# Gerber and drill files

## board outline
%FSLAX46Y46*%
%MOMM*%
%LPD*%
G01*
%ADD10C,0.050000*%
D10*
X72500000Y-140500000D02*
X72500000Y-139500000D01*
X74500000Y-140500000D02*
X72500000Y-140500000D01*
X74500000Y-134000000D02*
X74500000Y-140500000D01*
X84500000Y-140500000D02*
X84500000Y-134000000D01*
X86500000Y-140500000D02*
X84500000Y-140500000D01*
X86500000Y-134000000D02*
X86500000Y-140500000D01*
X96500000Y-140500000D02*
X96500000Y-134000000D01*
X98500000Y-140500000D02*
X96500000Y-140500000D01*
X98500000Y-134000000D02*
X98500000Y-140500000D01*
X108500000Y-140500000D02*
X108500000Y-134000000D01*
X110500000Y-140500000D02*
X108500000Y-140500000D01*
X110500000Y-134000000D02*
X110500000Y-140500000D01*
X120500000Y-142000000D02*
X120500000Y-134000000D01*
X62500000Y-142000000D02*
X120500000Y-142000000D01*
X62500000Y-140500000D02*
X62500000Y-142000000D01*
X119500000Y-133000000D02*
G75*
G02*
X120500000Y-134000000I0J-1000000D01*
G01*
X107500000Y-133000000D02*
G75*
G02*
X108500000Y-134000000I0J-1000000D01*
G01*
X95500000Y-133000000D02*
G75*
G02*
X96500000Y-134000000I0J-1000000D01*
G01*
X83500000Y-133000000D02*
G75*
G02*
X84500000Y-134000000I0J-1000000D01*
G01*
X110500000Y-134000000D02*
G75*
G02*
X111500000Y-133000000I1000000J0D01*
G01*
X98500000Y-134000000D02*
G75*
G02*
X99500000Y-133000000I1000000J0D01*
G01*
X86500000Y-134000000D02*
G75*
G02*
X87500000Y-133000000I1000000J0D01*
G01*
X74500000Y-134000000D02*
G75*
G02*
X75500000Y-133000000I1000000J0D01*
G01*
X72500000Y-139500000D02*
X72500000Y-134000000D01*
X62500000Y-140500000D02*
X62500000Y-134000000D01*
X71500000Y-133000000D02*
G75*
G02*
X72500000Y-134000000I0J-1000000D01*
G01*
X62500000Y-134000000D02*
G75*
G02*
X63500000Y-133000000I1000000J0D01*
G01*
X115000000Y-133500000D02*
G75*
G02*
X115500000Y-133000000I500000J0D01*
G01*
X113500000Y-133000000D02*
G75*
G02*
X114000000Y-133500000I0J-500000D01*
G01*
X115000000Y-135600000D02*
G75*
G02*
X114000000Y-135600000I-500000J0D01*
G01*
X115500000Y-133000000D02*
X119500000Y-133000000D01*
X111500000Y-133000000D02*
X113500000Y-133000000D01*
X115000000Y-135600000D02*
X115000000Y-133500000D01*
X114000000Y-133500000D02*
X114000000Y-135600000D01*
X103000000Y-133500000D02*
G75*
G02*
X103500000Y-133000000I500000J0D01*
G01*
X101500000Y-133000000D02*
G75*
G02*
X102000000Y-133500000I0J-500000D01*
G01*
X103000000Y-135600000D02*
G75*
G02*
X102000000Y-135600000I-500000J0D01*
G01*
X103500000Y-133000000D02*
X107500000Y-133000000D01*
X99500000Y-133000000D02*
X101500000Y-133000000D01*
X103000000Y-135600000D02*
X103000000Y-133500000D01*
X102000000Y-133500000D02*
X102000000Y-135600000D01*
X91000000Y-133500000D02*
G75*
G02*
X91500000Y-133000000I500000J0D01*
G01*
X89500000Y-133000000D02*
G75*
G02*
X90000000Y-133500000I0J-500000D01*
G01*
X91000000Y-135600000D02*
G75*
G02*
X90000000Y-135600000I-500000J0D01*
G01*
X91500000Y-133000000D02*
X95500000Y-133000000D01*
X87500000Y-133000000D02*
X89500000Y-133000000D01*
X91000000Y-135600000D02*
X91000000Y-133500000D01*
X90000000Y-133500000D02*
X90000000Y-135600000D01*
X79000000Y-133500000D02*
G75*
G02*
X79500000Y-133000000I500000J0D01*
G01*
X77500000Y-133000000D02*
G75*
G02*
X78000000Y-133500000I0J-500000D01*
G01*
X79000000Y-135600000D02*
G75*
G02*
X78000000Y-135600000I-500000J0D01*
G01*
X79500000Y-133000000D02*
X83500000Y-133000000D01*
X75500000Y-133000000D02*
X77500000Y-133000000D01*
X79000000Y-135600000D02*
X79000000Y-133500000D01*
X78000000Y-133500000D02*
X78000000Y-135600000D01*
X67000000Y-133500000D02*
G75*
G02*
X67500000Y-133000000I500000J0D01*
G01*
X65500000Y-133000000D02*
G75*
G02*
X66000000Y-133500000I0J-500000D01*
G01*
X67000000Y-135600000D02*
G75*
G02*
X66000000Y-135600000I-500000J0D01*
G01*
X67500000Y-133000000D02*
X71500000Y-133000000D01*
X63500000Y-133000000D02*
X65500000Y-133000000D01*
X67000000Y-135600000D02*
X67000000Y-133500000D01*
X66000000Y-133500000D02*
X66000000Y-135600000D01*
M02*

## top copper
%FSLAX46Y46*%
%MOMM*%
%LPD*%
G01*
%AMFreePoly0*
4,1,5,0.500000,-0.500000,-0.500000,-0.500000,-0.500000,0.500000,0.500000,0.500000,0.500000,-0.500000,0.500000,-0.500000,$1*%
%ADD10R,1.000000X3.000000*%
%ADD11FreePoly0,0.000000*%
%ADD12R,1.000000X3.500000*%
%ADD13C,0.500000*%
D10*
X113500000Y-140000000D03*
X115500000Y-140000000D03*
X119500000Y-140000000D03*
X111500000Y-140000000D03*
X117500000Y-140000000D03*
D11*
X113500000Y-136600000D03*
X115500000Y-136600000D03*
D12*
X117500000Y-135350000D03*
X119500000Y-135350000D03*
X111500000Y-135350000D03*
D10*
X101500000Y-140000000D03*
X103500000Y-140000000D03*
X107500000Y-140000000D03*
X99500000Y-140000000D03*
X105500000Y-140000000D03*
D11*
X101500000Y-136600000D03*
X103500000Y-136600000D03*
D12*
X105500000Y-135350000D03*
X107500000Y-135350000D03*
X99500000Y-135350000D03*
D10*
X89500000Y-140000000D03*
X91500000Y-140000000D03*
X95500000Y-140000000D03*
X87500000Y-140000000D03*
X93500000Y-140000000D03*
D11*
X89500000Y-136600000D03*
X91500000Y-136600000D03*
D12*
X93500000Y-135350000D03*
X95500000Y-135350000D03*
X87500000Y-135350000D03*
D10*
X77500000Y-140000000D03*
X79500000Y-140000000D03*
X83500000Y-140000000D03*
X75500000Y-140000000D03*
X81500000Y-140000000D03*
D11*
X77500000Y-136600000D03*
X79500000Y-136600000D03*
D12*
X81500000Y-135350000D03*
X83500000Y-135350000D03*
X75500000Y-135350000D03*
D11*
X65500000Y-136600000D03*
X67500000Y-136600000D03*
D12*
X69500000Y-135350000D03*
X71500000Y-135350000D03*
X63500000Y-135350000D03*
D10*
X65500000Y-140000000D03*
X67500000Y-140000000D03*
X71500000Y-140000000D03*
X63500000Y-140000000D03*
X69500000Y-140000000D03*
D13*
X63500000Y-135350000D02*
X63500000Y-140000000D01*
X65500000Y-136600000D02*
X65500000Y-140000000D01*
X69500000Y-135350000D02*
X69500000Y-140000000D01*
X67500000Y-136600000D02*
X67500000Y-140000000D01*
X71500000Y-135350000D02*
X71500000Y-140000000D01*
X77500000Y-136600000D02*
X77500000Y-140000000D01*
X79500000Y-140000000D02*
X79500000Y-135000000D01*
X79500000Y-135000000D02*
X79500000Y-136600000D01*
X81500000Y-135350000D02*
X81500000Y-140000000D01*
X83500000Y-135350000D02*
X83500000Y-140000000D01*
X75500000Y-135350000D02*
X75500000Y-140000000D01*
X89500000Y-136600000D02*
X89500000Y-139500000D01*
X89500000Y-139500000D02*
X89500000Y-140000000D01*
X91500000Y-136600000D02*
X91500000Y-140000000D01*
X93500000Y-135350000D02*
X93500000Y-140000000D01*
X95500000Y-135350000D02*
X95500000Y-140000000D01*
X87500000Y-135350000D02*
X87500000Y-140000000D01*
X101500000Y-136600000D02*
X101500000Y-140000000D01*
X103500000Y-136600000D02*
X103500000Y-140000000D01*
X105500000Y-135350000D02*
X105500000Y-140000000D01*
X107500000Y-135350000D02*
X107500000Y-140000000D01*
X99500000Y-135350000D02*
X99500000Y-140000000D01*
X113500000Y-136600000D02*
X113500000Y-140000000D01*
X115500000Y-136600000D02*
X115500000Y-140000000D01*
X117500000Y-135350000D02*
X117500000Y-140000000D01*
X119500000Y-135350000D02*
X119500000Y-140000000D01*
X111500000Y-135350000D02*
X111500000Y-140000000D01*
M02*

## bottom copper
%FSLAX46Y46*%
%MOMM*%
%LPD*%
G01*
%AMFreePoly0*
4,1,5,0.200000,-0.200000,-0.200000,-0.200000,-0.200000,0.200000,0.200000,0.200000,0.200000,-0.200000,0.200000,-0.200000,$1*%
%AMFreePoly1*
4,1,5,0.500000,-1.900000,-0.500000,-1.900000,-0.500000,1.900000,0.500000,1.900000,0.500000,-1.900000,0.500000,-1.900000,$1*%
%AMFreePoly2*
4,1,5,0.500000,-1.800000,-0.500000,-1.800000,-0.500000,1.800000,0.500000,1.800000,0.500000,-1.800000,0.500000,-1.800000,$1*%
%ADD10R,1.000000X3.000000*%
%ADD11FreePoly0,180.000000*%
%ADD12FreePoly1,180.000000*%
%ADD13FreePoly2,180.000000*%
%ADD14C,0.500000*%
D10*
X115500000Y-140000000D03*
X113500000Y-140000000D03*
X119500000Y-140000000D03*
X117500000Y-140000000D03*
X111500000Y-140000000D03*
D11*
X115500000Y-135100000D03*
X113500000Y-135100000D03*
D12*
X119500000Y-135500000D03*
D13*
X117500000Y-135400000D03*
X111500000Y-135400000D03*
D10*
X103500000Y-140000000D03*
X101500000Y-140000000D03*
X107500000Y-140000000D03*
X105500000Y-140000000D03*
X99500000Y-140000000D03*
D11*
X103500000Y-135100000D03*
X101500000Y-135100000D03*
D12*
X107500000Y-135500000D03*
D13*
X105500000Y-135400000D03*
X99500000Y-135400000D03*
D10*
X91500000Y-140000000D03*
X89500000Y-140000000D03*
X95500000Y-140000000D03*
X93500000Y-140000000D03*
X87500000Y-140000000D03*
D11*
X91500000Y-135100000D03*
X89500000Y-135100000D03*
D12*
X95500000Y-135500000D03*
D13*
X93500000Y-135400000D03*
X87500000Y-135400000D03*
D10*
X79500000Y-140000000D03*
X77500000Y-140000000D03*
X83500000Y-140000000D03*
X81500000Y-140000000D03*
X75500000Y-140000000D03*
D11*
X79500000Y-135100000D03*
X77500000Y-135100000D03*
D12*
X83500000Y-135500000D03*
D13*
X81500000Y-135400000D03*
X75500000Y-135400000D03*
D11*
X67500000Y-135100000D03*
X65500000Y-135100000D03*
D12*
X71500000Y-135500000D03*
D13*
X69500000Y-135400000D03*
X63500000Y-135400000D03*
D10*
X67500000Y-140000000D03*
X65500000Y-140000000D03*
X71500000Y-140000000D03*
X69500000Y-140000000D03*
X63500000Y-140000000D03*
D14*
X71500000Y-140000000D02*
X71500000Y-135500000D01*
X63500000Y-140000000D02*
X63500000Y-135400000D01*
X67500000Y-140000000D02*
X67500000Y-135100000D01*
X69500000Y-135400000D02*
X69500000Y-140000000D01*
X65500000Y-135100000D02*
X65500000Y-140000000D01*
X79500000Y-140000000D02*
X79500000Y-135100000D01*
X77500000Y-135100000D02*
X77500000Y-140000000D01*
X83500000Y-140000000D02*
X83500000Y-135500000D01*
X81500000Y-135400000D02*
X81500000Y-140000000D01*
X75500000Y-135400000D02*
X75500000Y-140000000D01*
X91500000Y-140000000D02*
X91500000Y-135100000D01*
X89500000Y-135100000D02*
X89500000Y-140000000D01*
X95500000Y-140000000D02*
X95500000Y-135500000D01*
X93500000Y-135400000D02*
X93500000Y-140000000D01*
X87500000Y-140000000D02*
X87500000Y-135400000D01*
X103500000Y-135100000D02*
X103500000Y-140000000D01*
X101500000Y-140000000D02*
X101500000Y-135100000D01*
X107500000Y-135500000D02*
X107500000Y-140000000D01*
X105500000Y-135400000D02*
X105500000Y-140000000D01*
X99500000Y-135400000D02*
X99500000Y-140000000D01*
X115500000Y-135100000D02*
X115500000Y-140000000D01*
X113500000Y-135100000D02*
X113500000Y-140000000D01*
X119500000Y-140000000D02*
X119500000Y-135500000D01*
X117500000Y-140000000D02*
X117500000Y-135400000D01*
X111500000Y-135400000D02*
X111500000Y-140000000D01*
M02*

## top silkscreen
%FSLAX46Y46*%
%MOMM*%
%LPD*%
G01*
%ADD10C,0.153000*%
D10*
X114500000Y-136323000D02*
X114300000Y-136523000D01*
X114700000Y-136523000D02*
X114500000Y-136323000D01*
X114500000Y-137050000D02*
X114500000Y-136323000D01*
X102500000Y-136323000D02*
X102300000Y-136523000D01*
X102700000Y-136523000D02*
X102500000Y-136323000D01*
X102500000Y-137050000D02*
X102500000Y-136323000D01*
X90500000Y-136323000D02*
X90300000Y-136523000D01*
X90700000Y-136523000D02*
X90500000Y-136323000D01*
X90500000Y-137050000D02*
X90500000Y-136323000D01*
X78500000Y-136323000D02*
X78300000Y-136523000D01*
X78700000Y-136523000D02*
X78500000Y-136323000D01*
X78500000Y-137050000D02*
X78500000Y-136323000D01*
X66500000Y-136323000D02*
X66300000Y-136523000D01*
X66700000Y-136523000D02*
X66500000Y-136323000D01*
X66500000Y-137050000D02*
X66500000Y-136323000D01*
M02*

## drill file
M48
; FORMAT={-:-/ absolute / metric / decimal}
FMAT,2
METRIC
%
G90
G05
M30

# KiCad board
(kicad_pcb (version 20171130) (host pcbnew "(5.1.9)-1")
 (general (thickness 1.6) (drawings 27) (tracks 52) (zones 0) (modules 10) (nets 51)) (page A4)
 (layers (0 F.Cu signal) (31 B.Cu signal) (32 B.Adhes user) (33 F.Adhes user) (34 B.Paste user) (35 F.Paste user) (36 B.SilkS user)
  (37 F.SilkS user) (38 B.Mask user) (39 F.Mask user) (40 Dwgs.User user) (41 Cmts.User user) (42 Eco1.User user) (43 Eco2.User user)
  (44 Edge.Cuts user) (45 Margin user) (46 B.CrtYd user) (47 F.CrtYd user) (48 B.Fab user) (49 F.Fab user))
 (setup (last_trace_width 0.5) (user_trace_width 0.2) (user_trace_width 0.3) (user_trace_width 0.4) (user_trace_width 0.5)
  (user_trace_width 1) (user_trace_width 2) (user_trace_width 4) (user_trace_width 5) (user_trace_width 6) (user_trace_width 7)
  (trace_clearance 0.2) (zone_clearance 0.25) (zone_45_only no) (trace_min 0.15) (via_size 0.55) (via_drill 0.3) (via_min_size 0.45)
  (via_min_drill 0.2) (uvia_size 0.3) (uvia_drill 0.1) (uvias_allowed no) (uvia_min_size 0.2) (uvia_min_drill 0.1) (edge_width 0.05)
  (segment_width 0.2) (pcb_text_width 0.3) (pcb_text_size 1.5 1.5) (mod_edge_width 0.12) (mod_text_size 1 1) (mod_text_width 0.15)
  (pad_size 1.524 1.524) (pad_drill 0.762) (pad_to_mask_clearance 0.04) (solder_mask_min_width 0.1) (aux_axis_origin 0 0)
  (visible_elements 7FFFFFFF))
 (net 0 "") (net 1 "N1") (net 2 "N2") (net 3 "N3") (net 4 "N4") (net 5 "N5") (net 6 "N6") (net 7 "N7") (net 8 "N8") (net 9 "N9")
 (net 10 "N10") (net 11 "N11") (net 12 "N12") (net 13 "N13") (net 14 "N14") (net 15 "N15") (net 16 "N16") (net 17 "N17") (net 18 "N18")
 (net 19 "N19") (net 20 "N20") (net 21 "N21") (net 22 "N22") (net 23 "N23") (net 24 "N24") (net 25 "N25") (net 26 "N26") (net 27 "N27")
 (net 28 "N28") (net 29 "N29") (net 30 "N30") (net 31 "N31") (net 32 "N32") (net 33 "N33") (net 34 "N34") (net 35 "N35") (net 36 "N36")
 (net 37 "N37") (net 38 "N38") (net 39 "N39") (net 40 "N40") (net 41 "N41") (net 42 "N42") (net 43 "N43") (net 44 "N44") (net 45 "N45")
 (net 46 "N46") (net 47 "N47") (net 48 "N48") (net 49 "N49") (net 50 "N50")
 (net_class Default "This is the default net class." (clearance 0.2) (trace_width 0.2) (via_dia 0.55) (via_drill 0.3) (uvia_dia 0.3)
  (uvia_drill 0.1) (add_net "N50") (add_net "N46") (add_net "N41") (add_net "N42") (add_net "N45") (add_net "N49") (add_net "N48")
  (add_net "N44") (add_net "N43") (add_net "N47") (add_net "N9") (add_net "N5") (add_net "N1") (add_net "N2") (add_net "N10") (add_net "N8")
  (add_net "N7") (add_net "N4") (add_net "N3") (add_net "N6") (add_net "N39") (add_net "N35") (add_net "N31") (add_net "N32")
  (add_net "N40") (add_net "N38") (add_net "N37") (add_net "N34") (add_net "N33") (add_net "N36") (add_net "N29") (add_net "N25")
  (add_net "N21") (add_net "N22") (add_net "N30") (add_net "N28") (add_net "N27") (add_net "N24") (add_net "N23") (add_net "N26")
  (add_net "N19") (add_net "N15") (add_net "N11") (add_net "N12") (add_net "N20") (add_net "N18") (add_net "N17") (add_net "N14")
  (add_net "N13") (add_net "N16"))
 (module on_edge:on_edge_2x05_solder (layer F.Cu) (at 115.5 140)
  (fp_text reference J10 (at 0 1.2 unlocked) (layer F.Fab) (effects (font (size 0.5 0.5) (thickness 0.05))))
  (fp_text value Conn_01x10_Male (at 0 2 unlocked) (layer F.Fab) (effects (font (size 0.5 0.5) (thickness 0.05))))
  (pad 2 smd rect (at -2 0) (size 1 3) (layers F.Cu F.Mask) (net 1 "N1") (zone_connect 0))
  (pad 3 smd rect (at 0 0) (size 1 3) (layers F.Cu F.Mask) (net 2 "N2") (zone_connect 0))
  (pad 8 smd rect (at 0 0) (size 1 3) (layers B.Cu B.Mask) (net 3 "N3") (zone_connect 0))
  (pad 7 smd rect (at -2 0) (size 1 3) (layers B.Cu B.Mask) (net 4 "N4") (zone_connect 0))
  (pad 10 smd rect (at 4 0) (size 1 3) (layers B.Cu B.Mask) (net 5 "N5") (zone_connect 0))
  (pad 9 smd rect (at 2 0) (size 1 3) (layers B.Cu B.Mask) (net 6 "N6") (zone_connect 0))
  (pad 6 smd rect (at -4 0) (size 1 3) (layers B.Cu B.Mask) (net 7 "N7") (zone_connect 0))
  (pad 5 smd rect (at 4 0 180) (size 1 3) (layers F.Cu F.Mask) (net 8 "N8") (zone_connect 0))
  (pad 1 smd rect (at -4 0 180) (size 1 3) (layers F.Cu F.Mask) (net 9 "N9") (zone_connect 0))
  (pad 4 smd rect (at 2 0 180) (size 1 3) (layers F.Cu F.Mask) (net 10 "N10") (zone_connect 0)))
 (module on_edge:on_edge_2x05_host (layer F.Cu) (at 115.5 133)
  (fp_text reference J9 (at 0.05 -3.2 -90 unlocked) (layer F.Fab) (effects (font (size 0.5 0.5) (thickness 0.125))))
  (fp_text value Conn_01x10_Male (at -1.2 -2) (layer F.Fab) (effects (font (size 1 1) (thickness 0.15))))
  (fp_arc (start 0 0.5) (end 0 0) (angle -90) (layer Edge.Cuts) (width 0.05))
  (fp_arc (start -2 0.5) (end -1.5 0.5) (angle -90) (layer Edge.Cuts) (width 0.05))
  (fp_arc (start -1 2.6) (end -1.5 2.6) (angle -180) (layer Edge.Cuts) (width 0.05))
  (fp_line (start 0 0) (end 4 0) (layer Edge.Cuts) (width 0.05))
  (fp_line (start -4 0) (end -2 0) (layer Edge.Cuts) (width 0.05))
  (fp_line (start -0.5 2.6) (end -0.5 0.5) (layer Edge.Cuts) (width 0.05))
  (fp_line (start -1.5 0.5) (end -1.5 2.6) (layer Edge.Cuts) (width 0.05))
  (fp_line (start -1 3.323) (end -1.2 3.523) (layer F.SilkS) (width 0.153))
  (fp_line (start -0.8 3.523) (end -1 3.323) (layer F.SilkS) (width 0.153))
  (fp_line (start -1 4.05) (end -1 3.323) (layer F.SilkS) (width 0.153))
  (pad 2 smd custom (at -2 3.6) (size 1 1) (layers F.Cu F.Mask) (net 1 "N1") (zone_connect 0) (options (clearance outline) (anchor rect))
   (primitives))
  (pad 3 smd custom (at 0 3.6) (size 1 1) (layers F.Cu F.Mask) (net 2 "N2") (zone_connect 0) (options (clearance outline) (anchor rect))
   (primitives))
  (pad 8 smd custom (at 0 2.1 180) (size 0.4 0.4) (layers B.Cu B.Mask) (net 3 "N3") (zone_connect 0)
   (options (clearance outline) (anchor rect)) (primitives))
  (pad 7 smd custom (at -2 2.1 180) (size 0.4 0.4) (layers B.Cu B.Mask) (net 4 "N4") (zone_connect 0)
   (options (clearance outline) (anchor rect)) (primitives))
  (pad 4 smd rect (at 2 2.35) (size 1 3.5) (layers F.Cu F.Mask) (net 10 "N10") (zone_connect 0))
  (pad 10 smd custom (at 4 2.5 180) (size 1 3.8) (layers B.Cu B.Mask) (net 5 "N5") (zone_connect 0)
   (options (clearance outline) (anchor rect)) (primitives))
  (pad 9 smd custom (at 2 2.4 180) (size 1 3.6) (layers B.Cu B.Mask) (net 6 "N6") (zone_connect 0)
   (options (clearance outline) (anchor rect)) (primitives))
  (pad 6 smd custom (at -4 2.4 180) (size 1 3.6) (layers B.Cu B.Mask) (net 7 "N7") (zone_connect 0)
   (options (clearance outline) (anchor rect)) (primitives))
  (pad 5 smd rect (at 4 2.35) (size 1 3.5) (layers F.Cu F.Mask) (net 8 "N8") (zone_connect 0))
  (pad 1 smd rect (at -4 2.35) (size 1 3.5) (layers F.Cu F.Mask) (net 9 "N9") (zone_connect 0)))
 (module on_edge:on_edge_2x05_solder (layer F.Cu) (at 103.5 140)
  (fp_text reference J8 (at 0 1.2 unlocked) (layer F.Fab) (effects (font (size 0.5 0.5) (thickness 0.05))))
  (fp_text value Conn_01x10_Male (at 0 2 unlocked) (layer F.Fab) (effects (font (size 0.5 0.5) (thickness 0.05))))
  (pad 2 smd rect (at -2 0) (size 1 3) (layers F.Cu F.Mask) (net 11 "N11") (zone_connect 0))
  (pad 3 smd rect (at 0 0) (size 1 3) (layers F.Cu F.Mask) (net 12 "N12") (zone_connect 0))
  (pad 8 smd rect (at 0 0) (size 1 3) (layers B.Cu B.Mask) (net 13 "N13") (zone_connect 0))
  (pad 7 smd rect (at -2 0) (size 1 3) (layers B.Cu B.Mask) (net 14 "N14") (zone_connect 0))
  (pad 10 smd rect (at 4 0) (size 1 3) (layers B.Cu B.Mask) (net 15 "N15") (zone_connect 0))
  (pad 9 smd rect (at 2 0) (size 1 3) (layers B.Cu B.Mask) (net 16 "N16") (zone_connect 0))
  (pad 6 smd rect (at -4 0) (size 1 3) (layers B.Cu B.Mask) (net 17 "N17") (zone_connect 0))
  (pad 5 smd rect (at 4 0 180) (size 1 3) (layers F.Cu F.Mask) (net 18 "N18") (zone_connect 0))
  (pad 1 smd rect (at -4 0 180) (size 1 3) (layers F.Cu F.Mask) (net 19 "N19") (zone_connect 0))
  (pad 4 smd rect (at 2 0 180) (size 1 3) (layers F.Cu F.Mask) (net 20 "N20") (zone_connect 0)))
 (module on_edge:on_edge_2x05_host (layer F.Cu) (at 103.5 133)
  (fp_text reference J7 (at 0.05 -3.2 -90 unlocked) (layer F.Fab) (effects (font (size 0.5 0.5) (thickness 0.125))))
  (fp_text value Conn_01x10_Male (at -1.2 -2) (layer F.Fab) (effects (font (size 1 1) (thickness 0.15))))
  (fp_arc (start 0 0.5) (end 0 0) (angle -90) (layer Edge.Cuts) (width 0.05))
  (fp_arc (start -2 0.5) (end -1.5 0.5) (angle -90) (layer Edge.Cuts) (width 0.05))
  (fp_arc (start -1 2.6) (end -1.5 2.6) (angle -180) (layer Edge.Cuts) (width 0.05))
  (fp_line (start 0 0) (end 4 0) (layer Edge.Cuts) (width 0.05))
  (fp_line (start -4 0) (end -2 0) (layer Edge.Cuts) (width 0.05))
  (fp_line (start -0.5 2.6) (end -0.5 0.5) (layer Edge.Cuts) (width 0.05))
  (fp_line (start -1.5 0.5) (end -1.5 2.6) (layer Edge.Cuts) (width 0.05))
  (fp_line (start -1 3.323) (end -1.2 3.523) (layer F.SilkS) (width 0.153))
  (fp_line (start -0.8 3.523) (end -1 3.323) (layer F.SilkS) (width 0.153))
  (fp_line (start -1 4.05) (end -1 3.323) (layer F.SilkS) (width 0.153))
  (pad 2 smd custom (at -2 3.6) (size 1 1) (layers F.Cu F.Mask) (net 11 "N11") (zone_connect 0) (options (clearance outline) (anchor rect))
   (primitives))
  (pad 3 smd custom (at 0 3.6) (size 1 1) (layers F.Cu F.Mask) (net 12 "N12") (zone_connect 0) (options (clearance outline) (anchor rect))
   (primitives))
  (pad 8 smd custom (at 0 2.1 180) (size 0.4 0.4) (layers B.Cu B.Mask) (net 13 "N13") (zone_connect 0)
   (options (clearance outline) (anchor rect)) (primitives))
  (pad 7 smd custom (at -2 2.1 180) (size 0.4 0.4) (layers B.Cu B.Mask) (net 14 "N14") (zone_connect 0)
   (options (clearance outline) (anchor rect)) (primitives))
  (pad 4 smd rect (at 2 2.35) (size 1 3.5) (layers F.Cu F.Mask) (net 20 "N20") (zone_connect 0))
  (pad 10 smd custom (at 4 2.5 180) (size 1 3.8) (layers B.Cu B.Mask) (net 15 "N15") (zone_connect 0)
   (options (clearance outline) (anchor rect)) (primitives))
  (pad 9 smd custom (at 2 2.4 180) (size 1 3.6) (layers B.Cu B.Mask) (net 16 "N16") (zone_connect 0)
   (options (clearance outline) (anchor rect)) (primitives))
  (pad 6 smd custom (at -4 2.4 180) (size 1 3.6) (layers B.Cu B.Mask) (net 17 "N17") (zone_connect 0)
   (options (clearance outline) (anchor rect)) (primitives))
  (pad 5 smd rect (at 4 2.35) (size 1 3.5) (layers F.Cu F.Mask) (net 18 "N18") (zone_connect 0))
  (pad 1 smd rect (at -4 2.35) (size 1 3.5) (layers F.Cu F.Mask) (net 19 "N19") (zone_connect 0)))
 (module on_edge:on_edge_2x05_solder (layer F.Cu) (at 91.5 140)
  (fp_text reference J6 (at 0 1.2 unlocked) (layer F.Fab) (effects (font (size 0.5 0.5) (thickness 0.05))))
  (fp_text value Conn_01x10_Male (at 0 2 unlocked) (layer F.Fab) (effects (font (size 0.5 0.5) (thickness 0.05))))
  (pad 2 smd rect (at -2 0) (size 1 3) (layers F.Cu F.Mask) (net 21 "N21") (zone_connect 0))
  (pad 3 smd rect (at 0 0) (size 1 3) (layers F.Cu F.Mask) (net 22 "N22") (zone_connect 0))
  (pad 8 smd rect (at 0 0) (size 1 3) (layers B.Cu B.Mask) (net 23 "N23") (zone_connect 0))
  (pad 7 smd rect (at -2 0) (size 1 3) (layers B.Cu B.Mask) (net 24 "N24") (zone_connect 0))
  (pad 10 smd rect (at 4 0) (size 1 3) (layers B.Cu B.Mask) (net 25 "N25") (zone_connect 0))
  (pad 9 smd rect (at 2 0) (size 1 3) (layers B.Cu B.Mask) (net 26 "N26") (zone_connect 0))
  (pad 6 smd rect (at -4 0) (size 1 3) (layers B.Cu B.Mask) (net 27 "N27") (zone_connect 0))
  (pad 5 smd rect (at 4 0 180) (size 1 3) (layers F.Cu F.Mask) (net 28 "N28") (zone_connect 0))
  (pad 1 smd rect (at -4 0 180) (size 1 3) (layers F.Cu F.Mask) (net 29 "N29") (zone_connect 0))
  (pad 4 smd rect (at 2 0 180) (size 1 3) (layers F.Cu F.Mask) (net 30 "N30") (zone_connect 0)))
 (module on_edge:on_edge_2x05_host (layer F.Cu) (at 91.5 133)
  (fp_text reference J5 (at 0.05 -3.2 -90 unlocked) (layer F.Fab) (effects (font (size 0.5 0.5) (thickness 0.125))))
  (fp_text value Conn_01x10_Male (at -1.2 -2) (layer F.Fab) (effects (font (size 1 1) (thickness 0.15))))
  (fp_arc (start 0 0.5) (end 0 0) (angle -90) (layer Edge.Cuts) (width 0.05))
  (fp_arc (start -2 0.5) (end -1.5 0.5) (angle -90) (layer Edge.Cuts) (width 0.05))
  (fp_arc (start -1 2.6) (end -1.5 2.6) (angle -180) (layer Edge.Cuts) (width 0.05))
  (fp_line (start 0 0) (end 4 0) (layer Edge.Cuts) (width 0.05))
  (fp_line (start -4 0) (end -2 0) (layer Edge.Cuts) (width 0.05))
  (fp_line (start -0.5 2.6) (end -0.5 0.5) (layer Edge.Cuts) (width 0.05))
  (fp_line (start -1.5 0.5) (end -1.5 2.6) (layer Edge.Cuts) (width 0.05))
  (fp_line (start -1 3.323) (end -1.2 3.523) (layer F.SilkS) (width 0.153))
  (fp_line (start -0.8 3.523) (end -1 3.323) (layer F.SilkS) (width 0.153))
  (fp_line (start -1 4.05) (end -1 3.323) (layer F.SilkS) (width 0.153))
  (pad 2 smd custom (at -2 3.6) (size 1 1) (layers F.Cu F.Mask) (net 21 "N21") (zone_connect 0) (options (clearance outline) (anchor rect))
   (primitives))
  (pad 3 smd custom (at 0 3.6) (size 1 1) (layers F.Cu F.Mask) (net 22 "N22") (zone_connect 0) (options (clearance outline) (anchor rect))
   (primitives))
  (pad 8 smd custom (at 0 2.1 180) (size 0.4 0.4) (layers B.Cu B.Mask) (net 23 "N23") (zone_connect 0)
   (options (clearance outline) (anchor rect)) (primitives))
  (pad 7 smd custom (at -2 2.1 180) (size 0.4 0.4) (layers B.Cu B.Mask) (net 24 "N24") (zone_connect 0)
   (options (clearance outline) (anchor rect)) (primitives))
  (pad 4 smd rect (at 2 2.35) (size 1 3.5) (layers F.Cu F.Mask) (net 30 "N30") (zone_connect 0))
  (pad 10 smd custom (at 4 2.5 180) (size 1 3.8) (layers B.Cu B.Mask) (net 25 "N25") (zone_connect 0)
   (options (clearance outline) (anchor rect)) (primitives))
  (pad 9 smd custom (at 2 2.4 180) (size 1 3.6) (layers B.Cu B.Mask) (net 26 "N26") (zone_connect 0)
   (options (clearance outline) (anchor rect)) (primitives))
  (pad 6 smd custom (at -4 2.4 180) (size 1 3.6) (layers B.Cu B.Mask) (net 27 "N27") (zone_connect 0)
   (options (clearance outline) (anchor rect)) (primitives))
  (pad 5 smd rect (at 4 2.35) (size 1 3.5) (layers F.Cu F.Mask) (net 28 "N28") (zone_connect 0))
  (pad 1 smd rect (at -4 2.35) (size 1 3.5) (layers F.Cu F.Mask) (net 29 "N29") (zone_connect 0)))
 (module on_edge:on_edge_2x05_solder (layer F.Cu) (at 79.5 140)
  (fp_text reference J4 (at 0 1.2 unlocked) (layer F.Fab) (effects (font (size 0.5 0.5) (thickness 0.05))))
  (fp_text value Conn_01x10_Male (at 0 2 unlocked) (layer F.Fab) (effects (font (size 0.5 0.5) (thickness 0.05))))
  (pad 2 smd rect (at -2 0) (size 1 3) (layers F.Cu F.Mask) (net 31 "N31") (zone_connect 0))
  (pad 3 smd rect (at 0 0) (size 1 3) (layers F.Cu F.Mask) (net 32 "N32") (zone_connect 0))
  (pad 8 smd rect (at 0 0) (size 1 3) (layers B.Cu B.Mask) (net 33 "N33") (zone_connect 0))
  (pad 7 smd rect (at -2 0) (size 1 3) (layers B.Cu B.Mask) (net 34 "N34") (zone_connect 0))
  (pad 10 smd rect (at 4 0) (size 1 3) (layers B.Cu B.Mask) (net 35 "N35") (zone_connect 0))
  (pad 9 smd rect (at 2 0) (size 1 3) (layers B.Cu B.Mask) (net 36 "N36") (zone_connect 0))
  (pad 6 smd rect (at -4 0) (size 1 3) (layers B.Cu B.Mask) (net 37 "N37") (zone_connect 0))
  (pad 5 smd rect (at 4 0 180) (size 1 3) (layers F.Cu F.Mask) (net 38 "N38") (zone_connect 0))
  (pad 1 smd rect (at -4 0 180) (size 1 3) (layers F.Cu F.Mask) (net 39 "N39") (zone_connect 0))
  (pad 4 smd rect (at 2 0 180) (size 1 3) (layers F.Cu F.Mask) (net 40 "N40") (zone_connect 0)))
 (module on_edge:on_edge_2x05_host (layer F.Cu) (at 79.5 133)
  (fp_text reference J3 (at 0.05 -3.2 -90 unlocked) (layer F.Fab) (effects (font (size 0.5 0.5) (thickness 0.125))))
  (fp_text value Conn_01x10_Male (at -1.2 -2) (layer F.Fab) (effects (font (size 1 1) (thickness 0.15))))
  (fp_arc (start 0 0.5) (end 0 0) (angle -90) (layer Edge.Cuts) (width 0.05))
  (fp_arc (start -2 0.5) (end -1.5 0.5) (angle -90) (layer Edge.Cuts) (width 0.05))
  (fp_arc (start -1 2.6) (end -1.5 2.6) (angle -180) (layer Edge.Cuts) (width 0.05))
  (fp_line (start 0 0) (end 4 0) (layer Edge.Cuts) (width 0.05))
  (fp_line (start -4 0) (end -2 0) (layer Edge.Cuts) (width 0.05))
  (fp_line (start -0.5 2.6) (end -0.5 0.5) (layer Edge.Cuts) (width 0.05))
  (fp_line (start -1.5 0.5) (end -1.5 2.6) (layer Edge.Cuts) (width 0.05))
  (fp_line (start -1 3.323) (end -1.2 3.523) (layer F.SilkS) (width 0.153))
  (fp_line (start -0.8 3.523) (end -1 3.323) (layer F.SilkS) (width 0.153))
  (fp_line (start -1 4.05) (end -1 3.323) (layer F.SilkS) (width 0.153))
  (pad 2 smd custom (at -2 3.6) (size 1 1) (layers F.Cu F.Mask) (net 31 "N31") (zone_connect 0) (options (clearance outline) (anchor rect))
   (primitives))
  (pad 3 smd custom (at 0 3.6) (size 1 1) (layers F.Cu F.Mask) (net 32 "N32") (zone_connect 0) (options (clearance outline) (anchor rect))
   (primitives))
  (pad 8 smd custom (at 0 2.1 180) (size 0.4 0.4) (layers B.Cu B.Mask) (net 33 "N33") (zone_connect 0)
   (options (clearance outline) (anchor rect)) (primitives))
  (pad 7 smd custom (at -2 2.1 180) (size 0.4 0.4) (layers B.Cu B.Mask) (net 34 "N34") (zone_connect 0)
   (options (clearance outline) (anchor rect)) (primitives))
  (pad 4 smd rect (at 2 2.35) (size 1 3.5) (layers F.Cu F.Mask) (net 40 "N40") (zone_connect 0))
  (pad 10 smd custom (at 4 2.5 180) (size 1 3.8) (layers B.Cu B.Mask) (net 35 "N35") (zone_connect 0)
   (options (clearance outline) (anchor rect)) (primitives))
  (pad 9 smd custom (at 2 2.4 180) (size 1 3.6) (layers B.Cu B.Mask) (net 36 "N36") (zone_connect 0)
   (options (clearance outline) (anchor rect)) (primitives))
  (pad 6 smd custom (at -4 2.4 180) (size 1 3.6) (layers B.Cu B.Mask) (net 37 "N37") (zone_connect 0)
   (options (clearance outline) (anchor rect)) (primitives))
  (pad 5 smd rect (at 4 2.35) (size 1 3.5) (layers F.Cu F.Mask) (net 38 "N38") (zone_connect 0))
  (pad 1 smd rect (at -4 2.35) (size 1 3.5) (layers F.Cu F.Mask) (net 39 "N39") (zone_connect 0)))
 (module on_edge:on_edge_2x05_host (layer F.Cu) (at 67.5 133)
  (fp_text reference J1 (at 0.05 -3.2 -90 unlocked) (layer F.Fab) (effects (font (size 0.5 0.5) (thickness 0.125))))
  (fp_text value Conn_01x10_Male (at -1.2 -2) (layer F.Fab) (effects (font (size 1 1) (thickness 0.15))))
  (fp_arc (start 0 0.5) (end 0 0) (angle -90) (layer Edge.Cuts) (width 0.05))
  (fp_arc (start -2 0.5) (end -1.5 0.5) (angle -90) (layer Edge.Cuts) (width 0.05))
  (fp_arc (start -1 2.6) (end -1.5 2.6) (angle -180) (layer Edge.Cuts) (width 0.05))
  (fp_line (start 0 0) (end 4 0) (layer Edge.Cuts) (width 0.05))
  (fp_line (start -4 0) (end -2 0) (layer Edge.Cuts) (width 0.05))
  (fp_line (start -0.5 2.6) (end -0.5 0.5) (layer Edge.Cuts) (width 0.05))
  (fp_line (start -1.5 0.5) (end -1.5 2.6) (layer Edge.Cuts) (width 0.05))
  (fp_line (start -1 3.323) (end -1.2 3.523) (layer F.SilkS) (width 0.153))
  (fp_line (start -0.8 3.523) (end -1 3.323) (layer F.SilkS) (width 0.153))
  (fp_line (start -1 4.05) (end -1 3.323) (layer F.SilkS) (width 0.153))
  (pad 2 smd custom (at -2 3.6) (size 1 1) (layers F.Cu F.Mask) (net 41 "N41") (zone_connect 0) (options (clearance outline) (anchor rect))
   (primitives))
  (pad 3 smd custom (at 0 3.6) (size 1 1) (layers F.Cu F.Mask) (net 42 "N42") (zone_connect 0) (options (clearance outline) (anchor rect))
   (primitives))
  (pad 8 smd custom (at 0 2.1 180) (size 0.4 0.4) (layers B.Cu B.Mask) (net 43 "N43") (zone_connect 0)
   (options (clearance outline) (anchor rect)) (primitives))
  (pad 7 smd custom (at -2 2.1 180) (size 0.4 0.4) (layers B.Cu B.Mask) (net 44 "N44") (zone_connect 0)
   (options (clearance outline) (anchor rect)) (primitives))
  (pad 4 smd rect (at 2 2.35) (size 1 3.5) (layers F.Cu F.Mask) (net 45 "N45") (zone_connect 0))
  (pad 10 smd custom (at 4 2.5 180) (size 1 3.8) (layers B.Cu B.Mask) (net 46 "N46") (zone_connect 0)
   (options (clearance outline) (anchor rect)) (primitives))
  (pad 9 smd custom (at 2 2.4 180) (size 1 3.6) (layers B.Cu B.Mask) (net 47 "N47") (zone_connect 0)
   (options (clearance outline) (anchor rect)) (primitives))
  (pad 6 smd custom (at -4 2.4 180) (size 1 3.6) (layers B.Cu B.Mask) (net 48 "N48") (zone_connect 0)
   (options (clearance outline) (anchor rect)) (primitives))
  (pad 5 smd rect (at 4 2.35) (size 1 3.5) (layers F.Cu F.Mask) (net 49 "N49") (zone_connect 0))
  (pad 1 smd rect (at -4 2.35) (size 1 3.5) (layers F.Cu F.Mask) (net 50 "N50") (zone_connect 0)))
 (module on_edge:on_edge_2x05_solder (layer F.Cu) (at 67.5 140)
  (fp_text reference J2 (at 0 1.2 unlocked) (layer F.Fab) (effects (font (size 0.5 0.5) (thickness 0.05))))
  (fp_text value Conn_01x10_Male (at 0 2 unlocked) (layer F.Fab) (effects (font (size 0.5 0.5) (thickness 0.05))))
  (pad 2 smd rect (at -2 0) (size 1 3) (layers F.Cu F.Mask) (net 41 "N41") (zone_connect 0))
  (pad 3 smd rect (at 0 0) (size 1 3) (layers F.Cu F.Mask) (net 42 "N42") (zone_connect 0))
  (pad 8 smd rect (at 0 0) (size 1 3) (layers B.Cu B.Mask) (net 43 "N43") (zone_connect 0))
  (pad 7 smd rect (at -2 0) (size 1 3) (layers B.Cu B.Mask) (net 44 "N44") (zone_connect 0))
  (pad 10 smd rect (at 4 0) (size 1 3) (layers B.Cu B.Mask) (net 46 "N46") (zone_connect 0))
  (pad 9 smd rect (at 2 0) (size 1 3) (layers B.Cu B.Mask) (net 47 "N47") (zone_connect 0))
  (pad 6 smd rect (at -4 0) (size 1 3) (layers B.Cu B.Mask) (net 48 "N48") (zone_connect 0))
  (pad 5 smd rect (at 4 0 180) (size 1 3) (layers F.Cu F.Mask) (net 49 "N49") (zone_connect 0))
  (pad 1 smd rect (at -4 0 180) (size 1 3) (layers F.Cu F.Mask) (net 50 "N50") (zone_connect 0))
  (pad 4 smd rect (at 2 0 180) (size 1 3) (layers F.Cu F.Mask) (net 45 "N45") (zone_connect 0)))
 (gr_line (start 72.5 140.5) (end 72.5 139.5) (layer Edge.Cuts) (width 0.05))
 (gr_line (start 74.5 140.5) (end 72.5 140.5) (layer Edge.Cuts) (width 0.05))
 (gr_line (start 74.5 134) (end 74.5 140.5) (layer Edge.Cuts) (width 0.05))
 (gr_line (start 84.5 140.5) (end 84.5 134) (layer Edge.Cuts) (width 0.05))
 (gr_line (start 86.5 140.5) (end 84.5 140.5) (layer Edge.Cuts) (width 0.05))
 (gr_line (start 86.5 134) (end 86.5 140.5) (layer Edge.Cuts) (width 0.05))
 (gr_line (start 96.5 140.5) (end 96.5 134) (layer Edge.Cuts) (width 0.05))
 (gr_line (start 98.5 140.5) (end 96.5 140.5) (layer Edge.Cuts) (width 0.05))
 (gr_line (start 98.5 134) (end 98.5 140.5) (layer Edge.Cuts) (width 0.05))
 (gr_line (start 108.5 140.5) (end 108.5 134) (layer Edge.Cuts) (width 0.05))
 (gr_line (start 110.5 140.5) (end 108.5 140.5) (layer Edge.Cuts) (width 0.05))
 (gr_line (start 110.5 134) (end 110.5 140.5) (layer Edge.Cuts) (width 0.05))
 (gr_line (start 120.5 142) (end 120.5 134) (layer Edge.Cuts) (width 0.05))
 (gr_line (start 62.5 142) (end 120.5 142) (layer Edge.Cuts) (width 0.05))
 (gr_line (start 62.5 140.5) (end 62.5 142) (layer Edge.Cuts) (width 0.05))
 (gr_arc (start 119.5 134) (end 120.5 134) (angle -90) (layer Edge.Cuts) (width 0.05))
 (gr_arc (start 107.5 134) (end 108.5 134) (angle -90) (layer Edge.Cuts) (width 0.05))
 (gr_arc (start 95.5 134) (end 96.5 134) (angle -90) (layer Edge.Cuts) (width 0.05))
 (gr_arc (start 83.5 134) (end 84.5 134) (angle -90) (layer Edge.Cuts) (width 0.05))
 (gr_arc (start 111.5 134) (end 111.5 133) (angle -90) (layer Edge.Cuts) (width 0.05))
 (gr_arc (start 99.5 134) (end 99.5 133) (angle -90) (layer Edge.Cuts) (width 0.05))
 (gr_arc (start 87.5 134) (end 87.5 133) (angle -90) (layer Edge.Cuts) (width 0.05))
 (gr_arc (start 75.5 134) (end 75.5 133) (angle -90) (layer Edge.Cuts) (width 0.05))
 (gr_line (start 72.5 139.5) (end 72.5 134) (layer Edge.Cuts) (width 0.05))
 (gr_line (start 62.5 140.5) (end 62.5 134) (layer Edge.Cuts) (width 0.05))
 (gr_arc (start 71.5 134) (end 72.5 134) (angle -90) (layer Edge.Cuts) (width 0.05))
 (gr_arc (start 63.5 134) (end 63.5 133) (angle -90) (layer Edge.Cuts) (width 0.05))
 (segment (start 63.5 135.35) (end 63.5 140) (width 0.5) (layer F.Cu) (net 50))
 (segment (start 65.5 136.6) (end 65.5 140) (width 0.5) (layer F.Cu) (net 41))
 (segment (start 69.5 135.35) (end 69.5 140) (width 0.5) (layer F.Cu) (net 45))
 (segment (start 67.5 136.6) (end 67.5 140) (width 0.5) (layer F.Cu) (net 42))
 (segment (start 71.5 135.35) (end 71.5 140) (width 0.5) (layer F.Cu) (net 49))
 (segment (start 71.5 140) (end 71.5 135.5) (width 0.5) (layer B.Cu) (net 46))
 (segment (start 63.5 140) (end 63.5 135.4) (width 0.5) (layer B.Cu) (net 48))
 (segment (start 67.5 140) (end 67.5 135.1) (width 0.5) (layer B.Cu) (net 43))
 (segment (start 69.5 135.4) (end 69.5 140) (width 0.5) (layer B.Cu) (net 47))
 (segment (start 65.5 135.1) (end 65.5 140) (width 0.5) (layer B.Cu) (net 44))
 (segment (start 77.5 136.6) (end 77.5 140) (width 0.5) (layer F.Cu) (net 31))
 (segment (start 79.5 140) (end 79.5 135) (width 0.5) (layer F.Cu) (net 32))
 (segment (start 79.5 135) (end 79.5 136.6) (width 0.5) (layer F.Cu) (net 32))
 (segment (start 79.5 140) (end 79.5 135.1) (width 0.5) (layer B.Cu) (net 33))
 (segment (start 77.5 135.1) (end 77.5 140) (width 0.5) (layer B.Cu) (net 34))
 (segment (start 81.5 135.35) (end 81.5 140) (width 0.5) (layer F.Cu) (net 40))
 (segment (start 83.5 140) (end 83.5 135.5) (width 0.5) (layer B.Cu) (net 35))
 (segment (start 81.5 135.4) (end 81.5 140) (width 0.5) (layer B.Cu) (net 36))
 (segment (start 75.5 135.4) (end 75.5 140) (width 0.5) (layer B.Cu) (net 37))
 (segment (start 83.5 135.35) (end 83.5 140) (width 0.5) (layer F.Cu) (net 38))
 (segment (start 75.5 135.35) (end 75.5 140) (width 0.5) (layer F.Cu) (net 39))
 (segment (start 89.5 136.6) (end 89.5 139.5) (width 0.5) (layer F.Cu) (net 21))
 (segment (start 89.5 139.5) (end 89.5 140) (width 0.5) (layer F.Cu) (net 21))
 (segment (start 91.5 136.6) (end 91.5 140) (width 0.5) (layer F.Cu) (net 22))
 (segment (start 91.5 140) (end 91.5 135.1) (width 0.5) (layer B.Cu) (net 23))
 (segment (start 89.5 135.1) (end 89.5 140) (width 0.5) (layer B.Cu) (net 24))
 (segment (start 93.5 135.35) (end 93.5 140) (width 0.5) (layer F.Cu) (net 30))
 (segment (start 95.5 140) (end 95.5 135.5) (width 0.5) (layer B.Cu) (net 25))
 (segment (start 93.5 135.4) (end 93.5 140) (width 0.5) (layer B.Cu) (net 26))
 (segment (start 87.5 140) (end 87.5 135.4) (width 0.5) (layer B.Cu) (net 27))
 (segment (start 95.5 135.35) (end 95.5 140) (width 0.5) (layer F.Cu) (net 28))
 (segment (start 87.5 135.35) (end 87.5 140) (width 0.5) (layer F.Cu) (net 29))
 (segment (start 101.5 136.6) (end 101.5 140) (width 0.5) (layer F.Cu) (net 11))
 (segment (start 103.5 136.6) (end 103.5 140) (width 0.5) (layer F.Cu) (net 12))
 (segment (start 103.5 135.1) (end 103.5 140) (width 0.5) (layer B.Cu) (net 13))
 (segment (start 101.5 140) (end 101.5 135.1) (width 0.5) (layer B.Cu) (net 14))
 (segment (start 105.5 135.35) (end 105.5 140) (width 0.5) (layer F.Cu) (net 20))
 (segment (start 107.5 135.5) (end 107.5 140) (width 0.5) (layer B.Cu) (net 15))
 (segment (start 105.5 135.4) (end 105.5 140) (width 0.5) (layer B.Cu) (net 16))
 (segment (start 99.5 135.4) (end 99.5 140) (width 0.5) (layer B.Cu) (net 17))
 (segment (start 107.5 135.35) (end 107.5 140) (width 0.5) (layer F.Cu) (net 18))
 (segment (start 99.5 135.35) (end 99.5 140) (width 0.5) (layer F.Cu) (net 19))
 (segment (start 113.5 136.6) (end 113.5 140) (width 0.5) (layer F.Cu) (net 1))
 (segment (start 115.5 136.6) (end 115.5 140) (width 0.5) (layer F.Cu) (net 2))
 (segment (start 115.5 135.1) (end 115.5 140) (width 0.5) (layer B.Cu) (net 3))
 (segment (start 113.5 135.1) (end 113.5 140) (width 0.5) (layer B.Cu) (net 4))
 (segment (start 117.5 135.35) (end 117.5 140) (width 0.5) (layer F.Cu) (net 10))
 (segment (start 119.5 140) (end 119.5 135.5) (width 0.5) (layer B.Cu) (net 5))
 (segment (start 117.5 140) (end 117.5 135.4) (width 0.5) (layer B.Cu) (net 6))
 (segment (start 111.5 135.4) (end 111.5 140) (width 0.5) (layer B.Cu) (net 7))
 (segment (start 119.5 135.35) (end 119.5 140) (width 0.5) (layer F.Cu) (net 8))
 (segment (start 111.5 135.35) (end 111.5 140) (width 0.5) (layer F.Cu) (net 9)))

